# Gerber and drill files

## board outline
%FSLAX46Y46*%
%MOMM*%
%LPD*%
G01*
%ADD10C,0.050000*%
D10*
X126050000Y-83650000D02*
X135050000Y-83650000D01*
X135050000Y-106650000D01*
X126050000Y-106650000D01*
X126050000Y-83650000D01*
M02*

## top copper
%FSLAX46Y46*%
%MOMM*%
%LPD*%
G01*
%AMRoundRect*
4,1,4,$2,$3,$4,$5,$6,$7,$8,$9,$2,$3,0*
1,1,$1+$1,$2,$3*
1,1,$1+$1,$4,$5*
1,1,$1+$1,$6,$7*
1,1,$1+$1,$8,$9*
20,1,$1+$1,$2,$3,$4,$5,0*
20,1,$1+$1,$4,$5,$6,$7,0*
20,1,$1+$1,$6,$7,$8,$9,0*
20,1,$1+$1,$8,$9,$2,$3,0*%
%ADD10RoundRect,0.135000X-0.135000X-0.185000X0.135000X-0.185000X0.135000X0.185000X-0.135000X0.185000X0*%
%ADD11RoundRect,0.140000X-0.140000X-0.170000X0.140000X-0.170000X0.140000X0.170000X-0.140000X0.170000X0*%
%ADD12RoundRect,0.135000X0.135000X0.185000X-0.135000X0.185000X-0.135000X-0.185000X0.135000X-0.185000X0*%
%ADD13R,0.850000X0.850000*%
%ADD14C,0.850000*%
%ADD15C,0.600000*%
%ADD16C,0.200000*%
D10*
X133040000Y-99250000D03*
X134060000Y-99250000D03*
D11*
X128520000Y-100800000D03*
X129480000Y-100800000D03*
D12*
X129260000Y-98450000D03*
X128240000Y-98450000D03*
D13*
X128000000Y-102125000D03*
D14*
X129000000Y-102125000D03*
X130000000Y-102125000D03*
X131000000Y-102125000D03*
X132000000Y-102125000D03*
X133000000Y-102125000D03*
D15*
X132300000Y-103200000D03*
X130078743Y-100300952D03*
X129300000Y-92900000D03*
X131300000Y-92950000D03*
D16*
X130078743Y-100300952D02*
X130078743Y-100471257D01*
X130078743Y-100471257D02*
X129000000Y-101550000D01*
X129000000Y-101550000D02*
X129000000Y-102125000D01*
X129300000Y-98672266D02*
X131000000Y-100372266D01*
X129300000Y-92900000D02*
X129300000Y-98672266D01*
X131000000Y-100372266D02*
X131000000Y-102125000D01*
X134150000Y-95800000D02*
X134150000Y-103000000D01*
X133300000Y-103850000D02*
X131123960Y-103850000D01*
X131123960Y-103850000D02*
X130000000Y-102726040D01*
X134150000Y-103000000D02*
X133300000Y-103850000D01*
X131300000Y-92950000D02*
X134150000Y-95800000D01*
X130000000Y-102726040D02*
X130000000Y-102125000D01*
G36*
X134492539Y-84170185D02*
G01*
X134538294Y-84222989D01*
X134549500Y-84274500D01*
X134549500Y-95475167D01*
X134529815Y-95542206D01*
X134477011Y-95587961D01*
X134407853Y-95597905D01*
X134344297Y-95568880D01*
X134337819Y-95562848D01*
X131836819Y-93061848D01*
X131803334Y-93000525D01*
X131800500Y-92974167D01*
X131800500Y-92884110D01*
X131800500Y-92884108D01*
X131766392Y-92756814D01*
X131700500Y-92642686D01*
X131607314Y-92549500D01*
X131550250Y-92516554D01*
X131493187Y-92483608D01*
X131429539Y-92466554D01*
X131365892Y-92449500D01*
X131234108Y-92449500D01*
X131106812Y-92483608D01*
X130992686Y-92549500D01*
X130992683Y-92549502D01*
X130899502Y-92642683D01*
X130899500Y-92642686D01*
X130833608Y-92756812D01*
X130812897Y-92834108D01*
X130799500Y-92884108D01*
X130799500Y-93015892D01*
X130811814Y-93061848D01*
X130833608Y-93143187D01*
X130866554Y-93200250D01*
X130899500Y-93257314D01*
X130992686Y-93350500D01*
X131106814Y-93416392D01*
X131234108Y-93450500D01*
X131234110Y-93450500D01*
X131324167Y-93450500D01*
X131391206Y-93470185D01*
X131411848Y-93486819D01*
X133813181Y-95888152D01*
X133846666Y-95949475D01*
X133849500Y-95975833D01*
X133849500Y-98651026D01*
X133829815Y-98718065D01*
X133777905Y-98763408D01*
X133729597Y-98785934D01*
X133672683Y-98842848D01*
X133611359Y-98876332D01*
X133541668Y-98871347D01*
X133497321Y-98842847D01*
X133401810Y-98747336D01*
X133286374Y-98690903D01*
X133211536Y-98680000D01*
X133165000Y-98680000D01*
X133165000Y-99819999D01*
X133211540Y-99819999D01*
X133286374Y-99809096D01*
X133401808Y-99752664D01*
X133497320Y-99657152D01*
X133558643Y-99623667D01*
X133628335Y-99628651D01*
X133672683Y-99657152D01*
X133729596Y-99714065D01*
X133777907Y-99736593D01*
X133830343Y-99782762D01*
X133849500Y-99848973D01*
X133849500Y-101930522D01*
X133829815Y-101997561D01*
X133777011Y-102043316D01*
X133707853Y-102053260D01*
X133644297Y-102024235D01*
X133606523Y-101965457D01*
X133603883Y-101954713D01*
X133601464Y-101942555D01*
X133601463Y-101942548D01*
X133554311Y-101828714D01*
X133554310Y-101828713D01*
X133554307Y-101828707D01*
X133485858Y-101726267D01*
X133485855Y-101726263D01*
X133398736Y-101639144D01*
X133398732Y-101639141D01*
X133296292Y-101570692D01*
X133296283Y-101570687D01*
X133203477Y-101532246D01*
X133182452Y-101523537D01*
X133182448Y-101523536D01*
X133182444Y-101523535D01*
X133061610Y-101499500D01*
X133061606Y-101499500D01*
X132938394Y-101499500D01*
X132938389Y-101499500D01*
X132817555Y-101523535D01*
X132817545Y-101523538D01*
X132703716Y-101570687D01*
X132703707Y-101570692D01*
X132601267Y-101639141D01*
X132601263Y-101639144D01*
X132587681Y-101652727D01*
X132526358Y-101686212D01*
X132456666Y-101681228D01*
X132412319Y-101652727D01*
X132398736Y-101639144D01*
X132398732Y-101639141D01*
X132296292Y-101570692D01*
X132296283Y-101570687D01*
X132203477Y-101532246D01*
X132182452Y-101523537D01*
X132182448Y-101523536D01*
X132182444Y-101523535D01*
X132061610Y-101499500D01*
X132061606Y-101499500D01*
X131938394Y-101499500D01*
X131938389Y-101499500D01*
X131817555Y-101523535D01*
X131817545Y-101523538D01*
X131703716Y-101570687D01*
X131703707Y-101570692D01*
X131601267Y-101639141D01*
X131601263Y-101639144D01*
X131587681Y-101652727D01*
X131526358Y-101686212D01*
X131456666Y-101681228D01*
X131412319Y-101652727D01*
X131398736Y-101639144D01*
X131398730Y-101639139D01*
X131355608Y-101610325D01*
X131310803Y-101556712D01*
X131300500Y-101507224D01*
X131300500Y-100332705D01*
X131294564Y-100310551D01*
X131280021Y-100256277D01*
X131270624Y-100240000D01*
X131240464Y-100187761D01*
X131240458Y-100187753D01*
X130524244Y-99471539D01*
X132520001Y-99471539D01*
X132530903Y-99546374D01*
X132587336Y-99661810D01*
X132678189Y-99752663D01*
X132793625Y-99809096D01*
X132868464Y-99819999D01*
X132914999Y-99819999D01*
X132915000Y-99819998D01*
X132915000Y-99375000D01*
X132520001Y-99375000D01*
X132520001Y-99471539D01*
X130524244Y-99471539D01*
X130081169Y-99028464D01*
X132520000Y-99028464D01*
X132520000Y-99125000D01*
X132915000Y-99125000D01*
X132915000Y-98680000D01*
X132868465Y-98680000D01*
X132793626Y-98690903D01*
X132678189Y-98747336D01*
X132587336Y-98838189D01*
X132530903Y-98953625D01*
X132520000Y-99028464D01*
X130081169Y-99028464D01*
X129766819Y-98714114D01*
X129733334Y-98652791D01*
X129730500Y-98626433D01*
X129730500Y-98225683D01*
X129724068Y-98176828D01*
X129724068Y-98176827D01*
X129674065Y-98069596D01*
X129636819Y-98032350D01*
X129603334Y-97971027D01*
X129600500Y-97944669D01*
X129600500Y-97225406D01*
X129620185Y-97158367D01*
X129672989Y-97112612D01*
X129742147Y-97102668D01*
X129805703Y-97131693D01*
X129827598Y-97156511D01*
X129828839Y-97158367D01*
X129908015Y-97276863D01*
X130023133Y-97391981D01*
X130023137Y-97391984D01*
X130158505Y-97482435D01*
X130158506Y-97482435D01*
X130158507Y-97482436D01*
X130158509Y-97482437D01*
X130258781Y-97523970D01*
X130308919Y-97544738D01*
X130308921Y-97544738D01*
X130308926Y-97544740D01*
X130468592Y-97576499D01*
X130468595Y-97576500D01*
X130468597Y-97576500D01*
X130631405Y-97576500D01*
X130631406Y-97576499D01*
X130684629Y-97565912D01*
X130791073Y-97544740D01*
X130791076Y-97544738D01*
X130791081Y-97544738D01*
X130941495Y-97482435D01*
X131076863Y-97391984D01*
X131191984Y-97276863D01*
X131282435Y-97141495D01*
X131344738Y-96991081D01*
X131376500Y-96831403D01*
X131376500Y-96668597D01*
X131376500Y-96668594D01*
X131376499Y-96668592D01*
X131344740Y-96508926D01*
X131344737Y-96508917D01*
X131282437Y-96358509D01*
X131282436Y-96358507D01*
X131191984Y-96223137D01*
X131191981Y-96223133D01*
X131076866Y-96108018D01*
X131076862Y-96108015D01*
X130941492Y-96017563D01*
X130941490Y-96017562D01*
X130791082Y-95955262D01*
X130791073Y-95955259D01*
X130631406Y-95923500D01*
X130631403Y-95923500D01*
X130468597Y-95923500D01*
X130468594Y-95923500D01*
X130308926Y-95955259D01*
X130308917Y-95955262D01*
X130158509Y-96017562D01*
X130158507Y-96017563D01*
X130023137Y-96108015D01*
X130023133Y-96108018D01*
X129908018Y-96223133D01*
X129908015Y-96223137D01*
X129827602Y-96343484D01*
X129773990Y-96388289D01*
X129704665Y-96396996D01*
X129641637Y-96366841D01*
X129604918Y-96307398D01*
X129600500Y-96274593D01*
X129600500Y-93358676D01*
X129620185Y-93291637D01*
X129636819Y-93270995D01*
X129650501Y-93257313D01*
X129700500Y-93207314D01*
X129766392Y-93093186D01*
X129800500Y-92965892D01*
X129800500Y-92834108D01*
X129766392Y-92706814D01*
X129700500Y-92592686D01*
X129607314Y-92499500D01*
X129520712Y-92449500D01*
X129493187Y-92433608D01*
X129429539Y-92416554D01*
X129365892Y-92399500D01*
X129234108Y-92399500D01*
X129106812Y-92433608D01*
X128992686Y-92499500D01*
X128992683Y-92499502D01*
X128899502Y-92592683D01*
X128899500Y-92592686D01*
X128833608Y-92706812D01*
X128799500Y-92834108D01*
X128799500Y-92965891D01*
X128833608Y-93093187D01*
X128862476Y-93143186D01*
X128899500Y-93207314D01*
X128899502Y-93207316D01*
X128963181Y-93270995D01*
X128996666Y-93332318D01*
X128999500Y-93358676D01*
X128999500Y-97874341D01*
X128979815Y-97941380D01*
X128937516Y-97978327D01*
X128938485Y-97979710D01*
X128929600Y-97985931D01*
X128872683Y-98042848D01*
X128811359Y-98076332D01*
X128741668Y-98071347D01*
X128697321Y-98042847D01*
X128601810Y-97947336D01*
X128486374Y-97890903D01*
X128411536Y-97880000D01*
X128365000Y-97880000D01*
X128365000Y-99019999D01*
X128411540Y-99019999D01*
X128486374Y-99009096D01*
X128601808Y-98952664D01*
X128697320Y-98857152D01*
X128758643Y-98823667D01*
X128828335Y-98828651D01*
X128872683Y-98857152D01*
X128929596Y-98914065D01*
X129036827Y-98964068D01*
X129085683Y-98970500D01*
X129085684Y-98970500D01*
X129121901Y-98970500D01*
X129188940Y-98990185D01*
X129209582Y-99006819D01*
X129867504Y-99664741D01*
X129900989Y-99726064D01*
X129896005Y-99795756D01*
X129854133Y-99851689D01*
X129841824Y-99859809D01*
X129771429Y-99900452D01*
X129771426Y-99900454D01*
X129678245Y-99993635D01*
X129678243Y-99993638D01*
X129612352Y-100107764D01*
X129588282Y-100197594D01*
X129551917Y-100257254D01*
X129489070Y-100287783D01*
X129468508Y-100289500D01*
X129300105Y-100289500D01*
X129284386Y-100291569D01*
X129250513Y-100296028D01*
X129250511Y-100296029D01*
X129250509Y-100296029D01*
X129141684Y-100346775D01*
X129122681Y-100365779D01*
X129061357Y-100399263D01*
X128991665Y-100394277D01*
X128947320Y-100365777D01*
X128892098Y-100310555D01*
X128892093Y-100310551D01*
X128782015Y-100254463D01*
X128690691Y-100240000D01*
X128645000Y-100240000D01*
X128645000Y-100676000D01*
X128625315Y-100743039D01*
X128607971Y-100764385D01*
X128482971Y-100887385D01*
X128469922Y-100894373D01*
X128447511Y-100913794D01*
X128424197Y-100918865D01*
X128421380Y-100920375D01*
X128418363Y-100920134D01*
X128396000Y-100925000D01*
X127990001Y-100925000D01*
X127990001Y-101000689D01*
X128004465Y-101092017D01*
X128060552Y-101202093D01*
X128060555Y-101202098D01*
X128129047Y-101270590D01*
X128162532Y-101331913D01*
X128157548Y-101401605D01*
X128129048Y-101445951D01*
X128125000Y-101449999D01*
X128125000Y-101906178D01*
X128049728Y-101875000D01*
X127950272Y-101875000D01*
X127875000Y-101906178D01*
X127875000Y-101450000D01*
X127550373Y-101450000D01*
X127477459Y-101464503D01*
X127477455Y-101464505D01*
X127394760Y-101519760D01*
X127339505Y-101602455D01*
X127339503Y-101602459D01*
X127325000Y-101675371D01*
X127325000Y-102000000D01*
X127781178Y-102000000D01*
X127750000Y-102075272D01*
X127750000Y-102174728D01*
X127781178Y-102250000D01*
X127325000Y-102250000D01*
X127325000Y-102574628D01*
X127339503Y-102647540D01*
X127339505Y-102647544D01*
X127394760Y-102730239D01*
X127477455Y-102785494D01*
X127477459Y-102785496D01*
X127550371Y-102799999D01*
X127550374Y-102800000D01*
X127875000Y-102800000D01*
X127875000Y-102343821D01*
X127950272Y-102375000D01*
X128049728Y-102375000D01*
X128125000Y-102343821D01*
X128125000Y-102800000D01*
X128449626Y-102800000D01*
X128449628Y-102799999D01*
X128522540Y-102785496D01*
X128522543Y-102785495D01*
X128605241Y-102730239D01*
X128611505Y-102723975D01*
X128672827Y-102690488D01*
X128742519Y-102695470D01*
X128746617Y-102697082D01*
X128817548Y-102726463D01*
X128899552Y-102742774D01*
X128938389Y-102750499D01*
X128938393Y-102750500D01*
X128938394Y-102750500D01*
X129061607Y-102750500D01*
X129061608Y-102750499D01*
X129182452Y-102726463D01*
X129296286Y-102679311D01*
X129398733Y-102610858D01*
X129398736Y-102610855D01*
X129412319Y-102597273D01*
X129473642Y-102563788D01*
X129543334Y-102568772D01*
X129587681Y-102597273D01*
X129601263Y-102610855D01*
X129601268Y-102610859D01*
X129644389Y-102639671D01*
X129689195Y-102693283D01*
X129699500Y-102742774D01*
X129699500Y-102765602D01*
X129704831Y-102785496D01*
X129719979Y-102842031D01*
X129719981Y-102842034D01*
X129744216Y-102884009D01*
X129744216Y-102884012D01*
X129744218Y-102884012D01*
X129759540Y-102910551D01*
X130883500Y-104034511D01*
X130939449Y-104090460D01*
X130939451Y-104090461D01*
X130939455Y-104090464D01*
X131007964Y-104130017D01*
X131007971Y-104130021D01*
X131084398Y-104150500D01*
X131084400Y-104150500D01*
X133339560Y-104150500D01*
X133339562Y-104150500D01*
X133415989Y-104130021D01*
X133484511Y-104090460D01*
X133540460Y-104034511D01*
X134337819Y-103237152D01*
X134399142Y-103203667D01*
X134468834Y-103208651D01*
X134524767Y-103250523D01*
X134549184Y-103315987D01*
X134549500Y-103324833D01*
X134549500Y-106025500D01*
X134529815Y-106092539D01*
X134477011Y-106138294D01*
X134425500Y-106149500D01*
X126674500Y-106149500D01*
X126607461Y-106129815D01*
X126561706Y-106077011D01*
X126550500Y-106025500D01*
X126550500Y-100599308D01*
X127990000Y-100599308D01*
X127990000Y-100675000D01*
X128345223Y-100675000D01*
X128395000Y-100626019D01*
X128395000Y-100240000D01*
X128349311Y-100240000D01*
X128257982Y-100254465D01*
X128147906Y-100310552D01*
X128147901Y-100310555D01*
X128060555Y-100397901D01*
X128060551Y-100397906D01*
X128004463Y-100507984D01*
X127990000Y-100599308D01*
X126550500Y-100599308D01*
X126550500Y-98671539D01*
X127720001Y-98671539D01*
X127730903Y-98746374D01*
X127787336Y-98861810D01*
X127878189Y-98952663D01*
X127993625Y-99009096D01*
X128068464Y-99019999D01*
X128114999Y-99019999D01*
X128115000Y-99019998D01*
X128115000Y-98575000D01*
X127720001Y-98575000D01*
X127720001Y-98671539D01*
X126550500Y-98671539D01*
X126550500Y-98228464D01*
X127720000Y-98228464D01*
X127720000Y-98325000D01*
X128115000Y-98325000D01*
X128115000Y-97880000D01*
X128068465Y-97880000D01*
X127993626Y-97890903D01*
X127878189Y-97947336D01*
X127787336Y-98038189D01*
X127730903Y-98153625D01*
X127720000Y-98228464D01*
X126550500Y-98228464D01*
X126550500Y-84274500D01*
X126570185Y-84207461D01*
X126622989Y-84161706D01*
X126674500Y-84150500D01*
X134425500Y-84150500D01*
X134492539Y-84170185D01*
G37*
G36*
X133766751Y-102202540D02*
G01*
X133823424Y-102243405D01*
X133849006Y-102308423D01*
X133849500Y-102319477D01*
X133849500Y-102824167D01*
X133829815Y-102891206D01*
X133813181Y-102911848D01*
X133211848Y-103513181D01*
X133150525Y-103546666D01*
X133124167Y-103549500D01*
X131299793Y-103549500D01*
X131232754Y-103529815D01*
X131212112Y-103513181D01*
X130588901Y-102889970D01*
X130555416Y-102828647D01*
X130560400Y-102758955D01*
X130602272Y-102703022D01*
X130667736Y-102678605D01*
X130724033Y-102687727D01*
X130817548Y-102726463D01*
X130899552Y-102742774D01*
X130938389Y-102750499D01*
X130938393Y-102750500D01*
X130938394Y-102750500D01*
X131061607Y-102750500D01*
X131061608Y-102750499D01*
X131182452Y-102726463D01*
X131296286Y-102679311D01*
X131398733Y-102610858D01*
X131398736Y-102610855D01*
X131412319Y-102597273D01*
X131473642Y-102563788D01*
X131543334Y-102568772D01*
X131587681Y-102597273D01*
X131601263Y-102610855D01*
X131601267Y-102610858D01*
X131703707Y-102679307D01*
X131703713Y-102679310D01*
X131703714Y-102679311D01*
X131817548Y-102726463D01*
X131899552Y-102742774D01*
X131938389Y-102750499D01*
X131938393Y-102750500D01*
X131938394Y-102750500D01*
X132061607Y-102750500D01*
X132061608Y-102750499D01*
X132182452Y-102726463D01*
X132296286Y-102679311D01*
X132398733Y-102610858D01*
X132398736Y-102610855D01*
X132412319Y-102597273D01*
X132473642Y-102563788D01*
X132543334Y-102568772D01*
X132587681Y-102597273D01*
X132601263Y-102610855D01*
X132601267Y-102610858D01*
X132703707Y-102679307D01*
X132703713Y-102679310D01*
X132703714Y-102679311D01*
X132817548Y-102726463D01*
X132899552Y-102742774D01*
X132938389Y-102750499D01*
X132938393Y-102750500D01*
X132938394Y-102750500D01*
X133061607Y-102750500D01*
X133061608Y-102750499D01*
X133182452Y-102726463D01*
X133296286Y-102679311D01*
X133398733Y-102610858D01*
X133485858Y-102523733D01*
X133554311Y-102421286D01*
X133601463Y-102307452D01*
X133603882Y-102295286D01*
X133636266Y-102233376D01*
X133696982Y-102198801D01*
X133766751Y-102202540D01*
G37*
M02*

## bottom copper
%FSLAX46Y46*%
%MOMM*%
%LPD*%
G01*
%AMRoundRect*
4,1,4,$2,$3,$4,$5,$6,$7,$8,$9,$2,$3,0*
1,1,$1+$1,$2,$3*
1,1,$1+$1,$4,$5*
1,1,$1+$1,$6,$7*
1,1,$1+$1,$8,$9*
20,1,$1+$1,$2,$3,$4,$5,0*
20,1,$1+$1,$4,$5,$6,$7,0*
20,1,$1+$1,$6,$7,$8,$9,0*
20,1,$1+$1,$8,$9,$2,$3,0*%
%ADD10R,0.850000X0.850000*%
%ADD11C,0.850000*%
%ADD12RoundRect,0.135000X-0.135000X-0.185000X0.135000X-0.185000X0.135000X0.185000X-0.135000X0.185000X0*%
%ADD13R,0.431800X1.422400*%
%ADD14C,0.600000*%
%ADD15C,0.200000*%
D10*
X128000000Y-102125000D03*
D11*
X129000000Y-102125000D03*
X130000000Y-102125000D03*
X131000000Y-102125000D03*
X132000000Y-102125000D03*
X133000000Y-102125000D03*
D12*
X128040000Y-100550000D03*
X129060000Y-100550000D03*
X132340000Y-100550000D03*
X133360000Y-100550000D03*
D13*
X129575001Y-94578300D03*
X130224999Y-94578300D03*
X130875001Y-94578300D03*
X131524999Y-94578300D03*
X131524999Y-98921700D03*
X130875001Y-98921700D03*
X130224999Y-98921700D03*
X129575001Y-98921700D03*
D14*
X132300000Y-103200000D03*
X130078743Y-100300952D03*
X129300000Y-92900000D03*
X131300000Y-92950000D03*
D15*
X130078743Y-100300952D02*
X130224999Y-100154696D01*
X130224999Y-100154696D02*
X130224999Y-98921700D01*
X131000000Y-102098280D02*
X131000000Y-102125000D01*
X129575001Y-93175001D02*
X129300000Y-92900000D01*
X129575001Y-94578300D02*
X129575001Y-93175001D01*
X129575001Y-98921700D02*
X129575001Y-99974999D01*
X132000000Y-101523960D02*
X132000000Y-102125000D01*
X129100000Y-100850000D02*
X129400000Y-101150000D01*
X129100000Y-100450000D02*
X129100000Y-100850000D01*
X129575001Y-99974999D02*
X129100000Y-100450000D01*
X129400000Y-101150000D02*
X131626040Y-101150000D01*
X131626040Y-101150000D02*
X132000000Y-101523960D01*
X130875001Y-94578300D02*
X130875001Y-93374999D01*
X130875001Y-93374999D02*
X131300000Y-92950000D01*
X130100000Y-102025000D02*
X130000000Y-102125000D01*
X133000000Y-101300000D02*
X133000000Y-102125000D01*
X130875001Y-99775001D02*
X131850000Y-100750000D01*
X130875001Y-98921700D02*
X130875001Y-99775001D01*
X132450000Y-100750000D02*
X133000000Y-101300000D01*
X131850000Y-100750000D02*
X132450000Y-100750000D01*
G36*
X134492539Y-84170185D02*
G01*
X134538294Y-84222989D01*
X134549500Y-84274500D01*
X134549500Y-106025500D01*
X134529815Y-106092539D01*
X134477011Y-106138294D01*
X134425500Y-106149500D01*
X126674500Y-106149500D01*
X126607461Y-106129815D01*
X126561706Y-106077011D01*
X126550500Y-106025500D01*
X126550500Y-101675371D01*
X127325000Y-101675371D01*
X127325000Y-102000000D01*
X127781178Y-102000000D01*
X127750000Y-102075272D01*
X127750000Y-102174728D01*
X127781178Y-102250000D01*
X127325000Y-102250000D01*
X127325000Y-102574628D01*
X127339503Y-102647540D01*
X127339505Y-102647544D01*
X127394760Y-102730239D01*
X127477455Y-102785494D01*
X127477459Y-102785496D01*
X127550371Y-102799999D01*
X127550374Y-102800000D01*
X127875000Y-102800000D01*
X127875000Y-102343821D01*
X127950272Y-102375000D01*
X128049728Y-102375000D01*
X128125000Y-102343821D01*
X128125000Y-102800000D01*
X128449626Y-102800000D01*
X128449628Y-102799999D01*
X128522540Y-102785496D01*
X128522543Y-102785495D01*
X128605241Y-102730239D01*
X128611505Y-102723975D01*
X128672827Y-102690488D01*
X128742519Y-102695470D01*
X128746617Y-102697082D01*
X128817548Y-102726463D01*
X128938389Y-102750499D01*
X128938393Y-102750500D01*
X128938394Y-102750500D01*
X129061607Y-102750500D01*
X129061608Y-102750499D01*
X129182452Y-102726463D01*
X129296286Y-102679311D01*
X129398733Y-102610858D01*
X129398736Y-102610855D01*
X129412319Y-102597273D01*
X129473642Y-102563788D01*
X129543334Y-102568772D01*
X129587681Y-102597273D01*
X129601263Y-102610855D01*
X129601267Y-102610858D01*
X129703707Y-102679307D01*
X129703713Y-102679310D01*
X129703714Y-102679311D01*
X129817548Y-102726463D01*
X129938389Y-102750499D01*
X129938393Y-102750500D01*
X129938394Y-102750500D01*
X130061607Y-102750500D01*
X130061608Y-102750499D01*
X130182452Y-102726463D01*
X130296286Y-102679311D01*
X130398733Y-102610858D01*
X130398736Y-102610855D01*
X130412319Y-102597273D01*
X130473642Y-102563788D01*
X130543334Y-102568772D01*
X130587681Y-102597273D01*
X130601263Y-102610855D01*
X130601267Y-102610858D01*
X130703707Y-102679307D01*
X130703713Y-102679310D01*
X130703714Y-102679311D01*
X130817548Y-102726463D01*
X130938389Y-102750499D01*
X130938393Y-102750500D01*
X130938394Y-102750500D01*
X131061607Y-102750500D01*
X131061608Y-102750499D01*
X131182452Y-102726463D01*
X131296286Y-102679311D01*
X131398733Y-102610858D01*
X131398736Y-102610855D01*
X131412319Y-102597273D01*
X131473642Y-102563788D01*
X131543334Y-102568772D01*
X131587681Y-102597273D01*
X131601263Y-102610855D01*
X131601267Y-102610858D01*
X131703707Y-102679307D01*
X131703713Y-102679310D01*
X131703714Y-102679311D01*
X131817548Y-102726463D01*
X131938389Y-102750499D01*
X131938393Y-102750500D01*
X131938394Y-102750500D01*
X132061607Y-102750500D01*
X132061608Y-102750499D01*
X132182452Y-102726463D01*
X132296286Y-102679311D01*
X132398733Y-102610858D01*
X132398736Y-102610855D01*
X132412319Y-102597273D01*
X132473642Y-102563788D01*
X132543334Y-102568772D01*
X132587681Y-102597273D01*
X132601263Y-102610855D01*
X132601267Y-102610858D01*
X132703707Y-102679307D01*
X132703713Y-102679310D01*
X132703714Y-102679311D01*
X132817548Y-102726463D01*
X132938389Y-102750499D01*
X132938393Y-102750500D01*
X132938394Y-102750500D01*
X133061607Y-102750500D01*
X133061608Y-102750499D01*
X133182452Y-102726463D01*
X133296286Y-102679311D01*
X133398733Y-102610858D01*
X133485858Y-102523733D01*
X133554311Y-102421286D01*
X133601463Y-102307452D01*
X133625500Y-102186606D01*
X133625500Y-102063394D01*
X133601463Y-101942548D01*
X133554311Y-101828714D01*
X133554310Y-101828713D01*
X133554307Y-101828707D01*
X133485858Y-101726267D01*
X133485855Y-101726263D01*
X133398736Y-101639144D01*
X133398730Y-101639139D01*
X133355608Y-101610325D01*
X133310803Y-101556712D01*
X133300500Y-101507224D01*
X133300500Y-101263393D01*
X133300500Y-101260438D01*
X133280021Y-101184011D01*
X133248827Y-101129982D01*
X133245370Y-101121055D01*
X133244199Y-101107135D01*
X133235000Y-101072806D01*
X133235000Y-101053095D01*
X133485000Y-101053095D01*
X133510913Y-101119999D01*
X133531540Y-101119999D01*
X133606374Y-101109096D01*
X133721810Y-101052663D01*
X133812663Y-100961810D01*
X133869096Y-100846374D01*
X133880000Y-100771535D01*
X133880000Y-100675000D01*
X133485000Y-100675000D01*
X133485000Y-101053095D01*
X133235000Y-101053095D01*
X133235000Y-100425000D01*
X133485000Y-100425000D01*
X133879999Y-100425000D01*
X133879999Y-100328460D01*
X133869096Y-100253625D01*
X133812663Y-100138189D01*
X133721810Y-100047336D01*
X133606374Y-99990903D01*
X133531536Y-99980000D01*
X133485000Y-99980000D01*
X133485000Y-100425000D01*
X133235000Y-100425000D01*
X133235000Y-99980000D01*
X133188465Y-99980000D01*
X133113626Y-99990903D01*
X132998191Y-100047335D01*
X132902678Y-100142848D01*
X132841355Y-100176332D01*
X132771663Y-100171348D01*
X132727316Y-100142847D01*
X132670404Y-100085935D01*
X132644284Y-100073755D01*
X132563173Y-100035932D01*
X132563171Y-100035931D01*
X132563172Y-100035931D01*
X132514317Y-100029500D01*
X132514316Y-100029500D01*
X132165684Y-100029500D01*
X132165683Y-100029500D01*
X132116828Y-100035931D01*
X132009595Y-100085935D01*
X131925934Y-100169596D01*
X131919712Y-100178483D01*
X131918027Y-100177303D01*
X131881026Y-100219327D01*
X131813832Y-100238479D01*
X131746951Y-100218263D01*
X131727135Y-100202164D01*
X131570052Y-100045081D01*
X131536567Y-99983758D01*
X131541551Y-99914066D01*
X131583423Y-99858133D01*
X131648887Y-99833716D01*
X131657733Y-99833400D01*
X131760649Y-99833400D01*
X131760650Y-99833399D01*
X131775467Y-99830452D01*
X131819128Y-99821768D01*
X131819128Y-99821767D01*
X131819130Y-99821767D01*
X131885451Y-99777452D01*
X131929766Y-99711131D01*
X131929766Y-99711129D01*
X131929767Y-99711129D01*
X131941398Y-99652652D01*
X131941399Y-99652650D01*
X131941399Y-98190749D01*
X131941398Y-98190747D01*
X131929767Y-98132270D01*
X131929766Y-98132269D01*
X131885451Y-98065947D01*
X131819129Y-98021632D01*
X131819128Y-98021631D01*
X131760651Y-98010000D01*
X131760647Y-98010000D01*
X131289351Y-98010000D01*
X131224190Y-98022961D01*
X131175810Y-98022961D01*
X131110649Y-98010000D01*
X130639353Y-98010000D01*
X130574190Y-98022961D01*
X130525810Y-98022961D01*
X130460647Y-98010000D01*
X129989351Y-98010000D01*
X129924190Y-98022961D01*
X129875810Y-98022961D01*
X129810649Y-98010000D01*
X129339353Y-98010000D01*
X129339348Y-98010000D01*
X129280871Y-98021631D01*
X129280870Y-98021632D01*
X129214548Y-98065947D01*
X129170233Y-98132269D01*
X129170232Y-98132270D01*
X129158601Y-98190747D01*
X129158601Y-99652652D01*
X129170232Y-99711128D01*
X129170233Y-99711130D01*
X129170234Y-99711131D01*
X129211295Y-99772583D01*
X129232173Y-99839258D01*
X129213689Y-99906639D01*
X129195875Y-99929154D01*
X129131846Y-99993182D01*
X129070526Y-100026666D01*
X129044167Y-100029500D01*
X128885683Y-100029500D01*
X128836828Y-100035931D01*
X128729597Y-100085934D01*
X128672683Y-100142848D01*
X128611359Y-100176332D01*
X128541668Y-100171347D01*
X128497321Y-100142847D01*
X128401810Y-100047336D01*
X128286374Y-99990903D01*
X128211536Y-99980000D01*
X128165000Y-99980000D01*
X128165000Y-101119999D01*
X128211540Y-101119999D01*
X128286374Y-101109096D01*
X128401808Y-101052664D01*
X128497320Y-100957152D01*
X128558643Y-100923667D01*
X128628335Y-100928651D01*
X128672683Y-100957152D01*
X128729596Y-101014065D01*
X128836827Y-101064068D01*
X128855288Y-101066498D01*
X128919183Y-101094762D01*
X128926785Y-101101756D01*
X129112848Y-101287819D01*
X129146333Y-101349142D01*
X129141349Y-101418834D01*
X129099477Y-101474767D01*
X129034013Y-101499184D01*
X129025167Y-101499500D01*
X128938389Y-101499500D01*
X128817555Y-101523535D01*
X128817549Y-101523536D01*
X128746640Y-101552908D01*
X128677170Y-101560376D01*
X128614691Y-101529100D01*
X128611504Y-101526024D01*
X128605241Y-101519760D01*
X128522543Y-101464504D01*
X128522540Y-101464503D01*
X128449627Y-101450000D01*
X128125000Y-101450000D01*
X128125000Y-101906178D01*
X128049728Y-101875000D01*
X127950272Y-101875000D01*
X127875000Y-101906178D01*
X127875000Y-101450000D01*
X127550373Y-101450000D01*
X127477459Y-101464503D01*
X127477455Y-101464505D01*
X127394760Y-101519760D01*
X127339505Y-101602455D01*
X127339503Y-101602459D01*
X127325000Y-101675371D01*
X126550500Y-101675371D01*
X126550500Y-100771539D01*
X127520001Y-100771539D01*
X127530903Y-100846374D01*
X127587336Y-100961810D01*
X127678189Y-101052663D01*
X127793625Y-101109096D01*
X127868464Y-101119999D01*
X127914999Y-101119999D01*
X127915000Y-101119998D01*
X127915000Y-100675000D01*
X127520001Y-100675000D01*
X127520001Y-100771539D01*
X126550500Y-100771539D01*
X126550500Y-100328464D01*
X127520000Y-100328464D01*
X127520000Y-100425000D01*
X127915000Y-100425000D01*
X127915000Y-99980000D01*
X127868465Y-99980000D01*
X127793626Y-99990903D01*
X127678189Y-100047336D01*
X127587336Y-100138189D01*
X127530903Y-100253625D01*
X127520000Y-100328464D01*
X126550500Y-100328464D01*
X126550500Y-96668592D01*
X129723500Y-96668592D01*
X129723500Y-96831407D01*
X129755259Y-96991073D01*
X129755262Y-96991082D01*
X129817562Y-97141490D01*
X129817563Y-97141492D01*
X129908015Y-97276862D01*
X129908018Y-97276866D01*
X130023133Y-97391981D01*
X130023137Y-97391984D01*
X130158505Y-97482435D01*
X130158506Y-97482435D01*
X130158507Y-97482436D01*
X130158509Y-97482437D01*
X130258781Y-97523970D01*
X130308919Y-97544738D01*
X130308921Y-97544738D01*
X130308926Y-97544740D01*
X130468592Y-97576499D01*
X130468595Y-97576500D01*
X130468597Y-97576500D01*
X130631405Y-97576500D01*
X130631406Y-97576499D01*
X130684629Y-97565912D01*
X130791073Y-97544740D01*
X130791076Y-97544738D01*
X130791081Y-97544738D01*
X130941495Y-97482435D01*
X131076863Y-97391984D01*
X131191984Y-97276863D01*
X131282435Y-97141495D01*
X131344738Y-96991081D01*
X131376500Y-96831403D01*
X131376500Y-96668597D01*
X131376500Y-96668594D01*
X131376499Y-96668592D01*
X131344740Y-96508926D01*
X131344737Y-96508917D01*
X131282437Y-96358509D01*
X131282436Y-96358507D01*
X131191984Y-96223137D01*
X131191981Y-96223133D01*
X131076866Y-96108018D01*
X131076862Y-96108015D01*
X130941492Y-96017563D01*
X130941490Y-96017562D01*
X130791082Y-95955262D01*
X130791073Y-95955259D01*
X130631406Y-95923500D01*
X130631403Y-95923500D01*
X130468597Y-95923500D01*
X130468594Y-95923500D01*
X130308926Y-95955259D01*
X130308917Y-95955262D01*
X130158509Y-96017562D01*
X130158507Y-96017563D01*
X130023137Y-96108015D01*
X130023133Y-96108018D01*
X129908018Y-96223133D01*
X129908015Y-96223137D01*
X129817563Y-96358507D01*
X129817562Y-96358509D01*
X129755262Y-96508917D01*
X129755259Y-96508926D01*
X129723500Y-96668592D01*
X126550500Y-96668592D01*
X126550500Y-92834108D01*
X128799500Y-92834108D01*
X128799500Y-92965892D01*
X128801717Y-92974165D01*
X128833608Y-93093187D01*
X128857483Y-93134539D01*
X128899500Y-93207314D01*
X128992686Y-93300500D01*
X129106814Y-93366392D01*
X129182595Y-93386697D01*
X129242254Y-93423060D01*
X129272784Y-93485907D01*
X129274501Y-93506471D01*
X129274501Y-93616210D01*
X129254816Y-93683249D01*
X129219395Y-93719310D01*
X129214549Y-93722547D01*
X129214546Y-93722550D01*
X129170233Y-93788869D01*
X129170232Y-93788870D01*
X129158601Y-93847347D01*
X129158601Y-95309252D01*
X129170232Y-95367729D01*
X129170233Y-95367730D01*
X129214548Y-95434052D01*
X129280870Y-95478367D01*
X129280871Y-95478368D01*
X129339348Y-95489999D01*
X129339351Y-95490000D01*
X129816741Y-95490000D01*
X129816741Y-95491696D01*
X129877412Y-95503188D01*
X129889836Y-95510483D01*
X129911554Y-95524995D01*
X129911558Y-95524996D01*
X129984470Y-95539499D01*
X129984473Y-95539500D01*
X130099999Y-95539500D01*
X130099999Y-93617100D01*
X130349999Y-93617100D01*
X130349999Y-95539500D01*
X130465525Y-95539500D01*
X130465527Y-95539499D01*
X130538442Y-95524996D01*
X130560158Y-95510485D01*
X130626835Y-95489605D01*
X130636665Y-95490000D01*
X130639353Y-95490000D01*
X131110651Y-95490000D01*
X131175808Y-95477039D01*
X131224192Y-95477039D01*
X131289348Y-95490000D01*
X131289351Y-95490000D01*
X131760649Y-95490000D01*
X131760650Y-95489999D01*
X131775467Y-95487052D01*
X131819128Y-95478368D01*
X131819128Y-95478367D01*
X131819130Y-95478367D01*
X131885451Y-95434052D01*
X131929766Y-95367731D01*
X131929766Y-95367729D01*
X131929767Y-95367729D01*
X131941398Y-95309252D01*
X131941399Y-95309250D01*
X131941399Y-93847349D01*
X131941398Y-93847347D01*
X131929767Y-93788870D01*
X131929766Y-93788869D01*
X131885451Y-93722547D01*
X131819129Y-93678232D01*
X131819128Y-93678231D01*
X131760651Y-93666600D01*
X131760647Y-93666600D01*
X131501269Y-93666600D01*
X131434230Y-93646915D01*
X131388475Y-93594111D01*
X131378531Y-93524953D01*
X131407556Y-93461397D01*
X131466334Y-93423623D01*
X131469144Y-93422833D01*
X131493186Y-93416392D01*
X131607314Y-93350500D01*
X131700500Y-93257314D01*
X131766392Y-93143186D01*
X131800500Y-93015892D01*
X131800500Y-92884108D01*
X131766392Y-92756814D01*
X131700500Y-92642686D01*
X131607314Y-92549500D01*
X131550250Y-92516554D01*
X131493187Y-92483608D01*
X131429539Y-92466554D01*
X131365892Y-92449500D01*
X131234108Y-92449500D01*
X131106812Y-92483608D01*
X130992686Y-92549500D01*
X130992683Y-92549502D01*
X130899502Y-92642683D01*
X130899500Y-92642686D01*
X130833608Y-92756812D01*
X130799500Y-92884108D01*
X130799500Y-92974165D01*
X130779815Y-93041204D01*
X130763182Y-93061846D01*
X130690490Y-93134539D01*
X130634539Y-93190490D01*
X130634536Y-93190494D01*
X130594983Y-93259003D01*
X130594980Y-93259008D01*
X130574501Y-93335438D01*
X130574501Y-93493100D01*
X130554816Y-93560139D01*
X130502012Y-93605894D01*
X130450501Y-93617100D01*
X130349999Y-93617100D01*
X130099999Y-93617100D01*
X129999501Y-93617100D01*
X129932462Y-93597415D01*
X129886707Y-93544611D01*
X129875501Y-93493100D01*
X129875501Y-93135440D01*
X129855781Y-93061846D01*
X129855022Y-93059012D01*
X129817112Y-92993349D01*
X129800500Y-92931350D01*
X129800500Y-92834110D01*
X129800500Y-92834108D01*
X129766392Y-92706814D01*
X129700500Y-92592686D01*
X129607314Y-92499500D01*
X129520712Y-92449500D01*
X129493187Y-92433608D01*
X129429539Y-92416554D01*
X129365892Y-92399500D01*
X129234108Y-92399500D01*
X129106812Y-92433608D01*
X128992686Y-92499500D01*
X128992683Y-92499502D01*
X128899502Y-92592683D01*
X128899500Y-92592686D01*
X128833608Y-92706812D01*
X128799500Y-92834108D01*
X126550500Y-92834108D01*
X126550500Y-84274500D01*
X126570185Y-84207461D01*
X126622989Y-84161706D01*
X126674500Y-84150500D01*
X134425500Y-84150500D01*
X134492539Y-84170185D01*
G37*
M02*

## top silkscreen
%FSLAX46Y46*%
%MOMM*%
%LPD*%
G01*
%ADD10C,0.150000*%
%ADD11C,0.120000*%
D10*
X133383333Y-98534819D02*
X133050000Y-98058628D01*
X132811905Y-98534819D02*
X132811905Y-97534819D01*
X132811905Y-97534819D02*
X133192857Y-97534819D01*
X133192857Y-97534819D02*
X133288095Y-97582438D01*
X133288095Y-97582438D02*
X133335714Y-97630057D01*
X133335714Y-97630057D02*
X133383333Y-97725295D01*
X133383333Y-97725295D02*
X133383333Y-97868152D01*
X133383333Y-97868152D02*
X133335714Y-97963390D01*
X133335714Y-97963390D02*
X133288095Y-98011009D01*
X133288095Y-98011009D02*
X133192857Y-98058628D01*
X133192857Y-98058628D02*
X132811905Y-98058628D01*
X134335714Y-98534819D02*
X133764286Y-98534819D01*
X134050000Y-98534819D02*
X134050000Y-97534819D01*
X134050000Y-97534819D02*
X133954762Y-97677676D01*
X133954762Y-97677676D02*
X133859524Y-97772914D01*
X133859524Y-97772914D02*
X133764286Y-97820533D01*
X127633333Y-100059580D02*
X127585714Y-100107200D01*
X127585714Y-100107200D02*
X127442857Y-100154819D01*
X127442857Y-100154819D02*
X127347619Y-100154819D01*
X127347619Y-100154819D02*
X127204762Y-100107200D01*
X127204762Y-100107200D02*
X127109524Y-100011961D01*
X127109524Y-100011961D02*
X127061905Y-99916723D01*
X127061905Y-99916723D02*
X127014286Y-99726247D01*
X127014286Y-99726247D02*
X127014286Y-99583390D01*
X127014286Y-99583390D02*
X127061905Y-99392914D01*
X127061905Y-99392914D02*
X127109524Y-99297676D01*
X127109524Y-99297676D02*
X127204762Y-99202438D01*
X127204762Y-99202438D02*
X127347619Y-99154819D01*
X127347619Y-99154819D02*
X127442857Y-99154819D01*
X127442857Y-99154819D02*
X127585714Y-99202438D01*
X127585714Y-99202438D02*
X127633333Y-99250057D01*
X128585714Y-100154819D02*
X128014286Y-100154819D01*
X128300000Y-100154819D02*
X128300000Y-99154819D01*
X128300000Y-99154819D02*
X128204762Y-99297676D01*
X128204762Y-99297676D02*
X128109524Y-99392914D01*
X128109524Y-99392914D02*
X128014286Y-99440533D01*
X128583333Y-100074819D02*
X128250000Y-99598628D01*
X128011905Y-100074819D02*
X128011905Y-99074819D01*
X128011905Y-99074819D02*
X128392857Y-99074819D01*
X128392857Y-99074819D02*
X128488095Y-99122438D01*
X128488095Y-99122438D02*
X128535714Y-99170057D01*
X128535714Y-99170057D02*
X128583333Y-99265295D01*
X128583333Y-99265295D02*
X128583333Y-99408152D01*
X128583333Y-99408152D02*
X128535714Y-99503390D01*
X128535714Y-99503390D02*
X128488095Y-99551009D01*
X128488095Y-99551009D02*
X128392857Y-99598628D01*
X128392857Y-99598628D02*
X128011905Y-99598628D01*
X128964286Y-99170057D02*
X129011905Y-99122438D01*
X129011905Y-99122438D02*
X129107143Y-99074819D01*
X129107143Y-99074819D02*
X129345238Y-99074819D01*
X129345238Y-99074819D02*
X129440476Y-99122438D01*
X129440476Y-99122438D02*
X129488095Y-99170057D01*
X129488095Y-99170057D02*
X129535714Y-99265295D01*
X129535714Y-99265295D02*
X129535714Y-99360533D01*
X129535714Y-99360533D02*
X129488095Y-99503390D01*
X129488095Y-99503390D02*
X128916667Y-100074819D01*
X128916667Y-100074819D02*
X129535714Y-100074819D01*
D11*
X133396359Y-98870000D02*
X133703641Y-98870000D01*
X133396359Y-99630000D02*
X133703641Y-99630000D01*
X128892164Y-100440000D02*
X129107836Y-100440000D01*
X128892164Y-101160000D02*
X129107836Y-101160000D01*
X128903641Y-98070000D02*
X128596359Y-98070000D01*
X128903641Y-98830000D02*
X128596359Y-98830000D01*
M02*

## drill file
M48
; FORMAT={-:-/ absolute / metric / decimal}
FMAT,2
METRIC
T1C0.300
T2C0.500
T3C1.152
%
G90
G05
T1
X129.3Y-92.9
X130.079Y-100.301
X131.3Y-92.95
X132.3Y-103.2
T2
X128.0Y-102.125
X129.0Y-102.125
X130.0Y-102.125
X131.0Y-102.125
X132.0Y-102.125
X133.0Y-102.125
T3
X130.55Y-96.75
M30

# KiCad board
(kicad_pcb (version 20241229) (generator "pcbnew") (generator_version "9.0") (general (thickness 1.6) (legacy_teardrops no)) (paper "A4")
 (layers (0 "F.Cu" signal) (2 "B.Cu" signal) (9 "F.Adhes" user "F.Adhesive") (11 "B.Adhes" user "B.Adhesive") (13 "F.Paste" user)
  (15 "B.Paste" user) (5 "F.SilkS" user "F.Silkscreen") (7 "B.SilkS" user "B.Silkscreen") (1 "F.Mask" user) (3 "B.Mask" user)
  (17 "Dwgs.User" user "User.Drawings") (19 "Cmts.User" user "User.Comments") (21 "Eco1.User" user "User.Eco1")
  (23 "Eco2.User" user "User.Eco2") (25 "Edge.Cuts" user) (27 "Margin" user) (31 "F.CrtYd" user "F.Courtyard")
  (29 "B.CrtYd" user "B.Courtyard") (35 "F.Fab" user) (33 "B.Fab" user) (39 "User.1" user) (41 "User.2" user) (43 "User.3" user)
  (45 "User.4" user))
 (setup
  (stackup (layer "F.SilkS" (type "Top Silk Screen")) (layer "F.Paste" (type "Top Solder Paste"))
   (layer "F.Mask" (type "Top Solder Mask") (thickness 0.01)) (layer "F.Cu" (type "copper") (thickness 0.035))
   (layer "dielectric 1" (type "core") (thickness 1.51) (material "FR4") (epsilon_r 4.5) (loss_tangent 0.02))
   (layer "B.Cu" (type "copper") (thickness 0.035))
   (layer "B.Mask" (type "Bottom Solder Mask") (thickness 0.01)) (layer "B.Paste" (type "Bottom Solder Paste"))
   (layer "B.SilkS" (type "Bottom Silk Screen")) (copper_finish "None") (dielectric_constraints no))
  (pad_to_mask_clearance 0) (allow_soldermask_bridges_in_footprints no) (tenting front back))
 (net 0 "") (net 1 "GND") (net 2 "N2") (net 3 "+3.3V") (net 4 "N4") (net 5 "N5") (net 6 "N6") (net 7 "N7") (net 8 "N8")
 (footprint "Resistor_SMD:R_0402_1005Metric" (layer "F.Cu") (at 133.55 99.25)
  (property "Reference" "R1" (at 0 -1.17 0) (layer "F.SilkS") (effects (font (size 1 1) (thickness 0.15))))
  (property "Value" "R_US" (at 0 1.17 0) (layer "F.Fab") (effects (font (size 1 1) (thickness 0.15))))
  (fp_line (start -0.153641 -0.38) (end 0.153641 -0.38) (stroke (width 0.12) (type solid)) (layer "F.SilkS"))
  (fp_line (start -0.153641 0.38) (end 0.153641 0.38) (stroke (width 0.12) (type solid)) (layer "F.SilkS"))
  (pad "1" smd roundrect (at -0.51 0) (size 0.54 0.64) (layers "F.Cu" "F.Mask" "F.Paste") (roundrect_rratio 0.25) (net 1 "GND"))
  (pad "2" smd roundrect (at 0.51 0) (size 0.54 0.64) (layers "F.Cu" "F.Mask" "F.Paste") (roundrect_rratio 0.25) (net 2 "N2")))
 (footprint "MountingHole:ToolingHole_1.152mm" (layer "F.Cu") (at 130.55 96.75)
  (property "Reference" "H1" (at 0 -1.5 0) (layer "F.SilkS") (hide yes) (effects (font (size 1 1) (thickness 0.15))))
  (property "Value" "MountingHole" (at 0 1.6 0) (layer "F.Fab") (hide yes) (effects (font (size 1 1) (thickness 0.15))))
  (pad "" np_thru_hole circle (at 0 0) (size 1.152 1.152) (drill 1.152) (layers "*.Cu" "*.Mask") (solder_mask_margin 0.074))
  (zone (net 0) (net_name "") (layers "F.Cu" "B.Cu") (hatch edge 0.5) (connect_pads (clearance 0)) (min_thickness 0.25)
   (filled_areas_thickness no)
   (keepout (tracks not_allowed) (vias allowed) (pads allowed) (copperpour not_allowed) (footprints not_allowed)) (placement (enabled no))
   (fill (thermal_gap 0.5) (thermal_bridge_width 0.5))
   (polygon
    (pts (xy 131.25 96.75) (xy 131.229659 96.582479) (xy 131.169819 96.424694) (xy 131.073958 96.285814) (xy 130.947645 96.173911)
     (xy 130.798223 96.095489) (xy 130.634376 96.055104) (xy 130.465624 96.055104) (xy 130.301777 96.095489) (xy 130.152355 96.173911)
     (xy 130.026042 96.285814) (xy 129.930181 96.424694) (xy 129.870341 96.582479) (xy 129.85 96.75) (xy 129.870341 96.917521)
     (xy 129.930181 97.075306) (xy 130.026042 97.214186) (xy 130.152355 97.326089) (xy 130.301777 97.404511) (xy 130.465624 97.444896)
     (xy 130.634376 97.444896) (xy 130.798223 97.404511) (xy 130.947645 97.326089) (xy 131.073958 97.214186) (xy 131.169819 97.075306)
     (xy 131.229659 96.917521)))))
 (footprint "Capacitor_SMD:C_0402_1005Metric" (layer "F.Cu") (at 129 100.8)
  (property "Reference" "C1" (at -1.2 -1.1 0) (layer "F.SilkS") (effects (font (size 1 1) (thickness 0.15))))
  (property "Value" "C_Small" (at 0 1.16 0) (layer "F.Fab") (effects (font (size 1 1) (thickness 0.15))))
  (fp_line (start -0.107836 -0.36) (end 0.107836 -0.36) (stroke (width 0.12) (type solid)) (layer "F.SilkS"))
  (fp_line (start -0.107836 0.36) (end 0.107836 0.36) (stroke (width 0.12) (type solid)) (layer "F.SilkS"))
  (pad "1" smd roundrect (at -0.48 0) (size 0.56 0.62) (layers "F.Cu" "F.Mask" "F.Paste") (roundrect_rratio 0.25) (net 1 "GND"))
  (pad "2" smd roundrect (at 0.48 0) (size 0.56 0.62) (layers "F.Cu" "F.Mask" "F.Paste") (roundrect_rratio 0.25) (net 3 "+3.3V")))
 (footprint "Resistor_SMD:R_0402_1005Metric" (layer "F.Cu") (at 128.75 98.45 180)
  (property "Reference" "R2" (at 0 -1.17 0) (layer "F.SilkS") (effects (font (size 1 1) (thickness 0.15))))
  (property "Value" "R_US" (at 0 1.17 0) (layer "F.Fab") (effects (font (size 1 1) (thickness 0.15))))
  (fp_line (start -0.153641 0.38) (end 0.153641 0.38) (stroke (width 0.12) (type solid)) (layer "F.SilkS"))
  (fp_line (start -0.153641 -0.38) (end 0.153641 -0.38) (stroke (width 0.12) (type solid)) (layer "F.SilkS"))
  (pad "1" smd roundrect (at -0.51 0 180) (size 0.54 0.64) (layers "F.Cu" "F.Mask" "F.Paste") (roundrect_rratio 0.25) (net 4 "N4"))
  (pad "2" smd roundrect (at 0.51 0 180) (size 0.54 0.64) (layers "F.Cu" "F.Mask" "F.Paste") (roundrect_rratio 0.25) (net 1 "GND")))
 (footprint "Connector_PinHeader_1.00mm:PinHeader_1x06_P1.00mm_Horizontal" (layer "B.Cu") (at 128 102.125 -90)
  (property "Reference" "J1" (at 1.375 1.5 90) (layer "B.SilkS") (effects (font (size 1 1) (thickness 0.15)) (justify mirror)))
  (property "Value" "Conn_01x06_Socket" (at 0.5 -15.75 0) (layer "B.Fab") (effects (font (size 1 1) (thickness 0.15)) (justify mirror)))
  (pad "1" thru_hole rect (at 0 0 270) (size 0.85 0.85) (drill 0.5) (layers "*.Cu" "*.Mask") (remove_unused_layers no) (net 1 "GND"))
  (pad "2" thru_hole circle (at 0 -1 270) (size 0.85 0.85) (drill 0.5) (layers "*.Cu" "*.Mask") (remove_unused_layers no) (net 3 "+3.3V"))
  (pad "3" thru_hole circle (at 0 -2 270) (size 0.85 0.85) (drill 0.5) (layers "*.Cu" "*.Mask") (remove_unused_layers no) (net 2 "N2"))
  (pad "4" thru_hole circle (at 0 -3 270) (size 0.85 0.85) (drill 0.5) (layers "*.Cu" "*.Mask") (remove_unused_layers no) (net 4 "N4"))
  (pad "5" thru_hole circle (at 0 -4 270) (size 0.85 0.85) (drill 0.5) (layers "*.Cu" "*.Mask") (remove_unused_layers no) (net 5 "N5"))
  (pad "6" thru_hole circle (at 0 -5 270) (size 0.85 0.85) (drill 0.5) (layers "*.Cu" "*.Mask") (remove_unused_layers no) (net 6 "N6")))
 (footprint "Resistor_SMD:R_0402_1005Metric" (layer "B.Cu") (at 128.55 100.55)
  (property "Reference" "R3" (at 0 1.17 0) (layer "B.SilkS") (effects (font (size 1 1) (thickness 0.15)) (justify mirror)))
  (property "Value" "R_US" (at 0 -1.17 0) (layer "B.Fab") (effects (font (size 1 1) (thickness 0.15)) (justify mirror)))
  (pad "1" smd roundrect (at -0.51 0) (size 0.54 0.64) (layers "B.Cu" "B.Mask" "B.Paste") (roundrect_rratio 0.25) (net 1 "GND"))
  (pad "2" smd roundrect (at 0.51 0) (size 0.54 0.64) (layers "B.Cu" "B.Mask" "B.Paste") (roundrect_rratio 0.25) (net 5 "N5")))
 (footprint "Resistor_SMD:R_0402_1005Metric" (layer "B.Cu") (at 132.85 100.55)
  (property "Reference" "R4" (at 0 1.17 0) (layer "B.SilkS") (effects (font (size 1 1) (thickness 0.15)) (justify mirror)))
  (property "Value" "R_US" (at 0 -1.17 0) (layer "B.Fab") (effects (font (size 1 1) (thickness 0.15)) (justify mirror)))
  (pad "1" smd roundrect (at -0.51 0) (size 0.54 0.64) (layers "B.Cu" "B.Mask" "B.Paste") (roundrect_rratio 0.25) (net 6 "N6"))
  (pad "2" smd roundrect (at 0.51 0) (size 0.54 0.64) (layers "B.Cu" "B.Mask" "B.Paste") (roundrect_rratio 0.25) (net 1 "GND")))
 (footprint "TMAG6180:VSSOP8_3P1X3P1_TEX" (layer "B.Cu") (at 130.55 96.75 -90)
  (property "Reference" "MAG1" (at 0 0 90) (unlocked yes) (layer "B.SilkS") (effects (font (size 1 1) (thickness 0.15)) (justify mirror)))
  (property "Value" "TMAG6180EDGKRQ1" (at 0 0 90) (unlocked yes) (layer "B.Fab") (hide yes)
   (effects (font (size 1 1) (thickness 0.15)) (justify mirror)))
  (pad "1" smd rect (at -2.1717 0.974999 270) (size 1.4224 0.4318) (layers "B.Cu" "B.Mask" "B.Paste") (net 4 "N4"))
  (pad "2" smd rect (at -2.1717 0.325001 270) (size 1.4224 0.4318) (layers "B.Cu" "B.Mask" "B.Paste") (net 1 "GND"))
  (pad "3" smd rect (at -2.1717 -0.325001 270) (size 1.4224 0.4318) (layers "B.Cu" "B.Mask" "B.Paste") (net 2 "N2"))
  (pad "4" smd rect (at -2.1717 -0.974999 270) (size 1.4224 0.4318) (layers "B.Cu" "B.Mask" "B.Paste") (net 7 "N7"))
  (pad "5" smd rect (at 2.1717 -0.974999 270) (size 1.4224 0.4318) (layers "B.Cu" "B.Mask" "B.Paste") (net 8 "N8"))
  (pad "6" smd rect (at 2.1717 -0.325001 270) (size 1.4224 0.4318) (layers "B.Cu" "B.Mask" "B.Paste") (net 6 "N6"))
  (pad "7" smd rect (at 2.1717 0.325001 270) (size 1.4224 0.4318) (layers "B.Cu" "B.Mask" "B.Paste") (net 3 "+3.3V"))
  (pad "8" smd rect (at 2.1717 0.974999 270) (size 1.4224 0.4318) (layers "B.Cu" "B.Mask" "B.Paste") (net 5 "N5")))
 (gr_rect (start 126.05 83.65) (end 135.05 106.65) (stroke (width 0.05) (type solid)) (fill no) (locked yes) (layer "Edge.Cuts"))
 (via (at 132.3 103.2) (size 0.6) (drill 0.3) (layers "F.Cu" "B.Cu") (free yes) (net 1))
 (segment (start 130.078743 100.300952) (end 130.078743 100.471257) (width 0.2) (layer "F.Cu") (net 3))
 (segment (start 130.078743 100.471257) (end 129 101.55) (width 0.2) (layer "F.Cu") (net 3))
 (segment (start 129 101.55) (end 129 102.125) (width 0.2) (layer "F.Cu") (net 3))
 (via (at 130.078743 100.300952) (size 0.6) (drill 0.3) (layers "F.Cu" "B.Cu") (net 3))
 (segment (start 130.078743 100.300952) (end 130.224999 100.154696) (width 0.2) (layer "B.Cu") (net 3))
 (segment (start 130.224999 100.154696) (end 130.224999 98.9217) (width 0.2) (layer "B.Cu") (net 3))
 (segment (start 129.3 98.672266) (end 131 100.372266) (width 0.2) (layer "F.Cu") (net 4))
 (segment (start 129.3 92.9) (end 129.3 98.672266) (width 0.2) (layer "F.Cu") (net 4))
 (segment (start 131 100.372266) (end 131 102.125) (width 0.2) (layer "F.Cu") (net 4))
 (via (at 129.3 92.9) (size 0.6) (drill 0.3) (layers "F.Cu" "B.Cu") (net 4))
 (segment (start 131 102.09828) (end 131 102.125) (width 0.2) (layer "B.Cu") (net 4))
 (segment (start 129.575001 93.175001) (end 129.3 92.9) (width 0.2) (layer "B.Cu") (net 4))
 (segment (start 129.575001 94.5783) (end 129.575001 93.175001) (width 0.2) (layer "B.Cu") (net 4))
 (segment (start 129.575001 98.9217) (end 129.575001 99.974999) (width 0.2) (layer "B.Cu") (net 5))
 (segment (start 132 101.52396) (end 132 102.125) (width 0.2) (layer "B.Cu") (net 5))
 (segment (start 129.1 100.85) (end 129.4 101.15) (width 0.2) (layer "B.Cu") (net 5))
 (segment (start 129.1 100.45) (end 129.1 100.85) (width 0.2) (layer "B.Cu") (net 5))
 (segment (start 129.575001 99.974999) (end 129.1 100.45) (width 0.2) (layer "B.Cu") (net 5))
 (segment (start 129.4 101.15) (end 131.62604 101.15) (width 0.2) (layer "B.Cu") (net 5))
 (segment (start 131.62604 101.15) (end 132 101.52396) (width 0.2) (layer "B.Cu") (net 5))
 (segment (start 134.15 95.8) (end 134.15 103) (width 0.2) (layer "F.Cu") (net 2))
 (segment (start 133.3 103.85) (end 131.12396 103.85) (width 0.2) (layer "F.Cu") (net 2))
 (segment (start 131.12396 103.85) (end 130 102.72604) (width 0.2) (layer "F.Cu") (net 2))
 (segment (start 134.15 103) (end 133.3 103.85) (width 0.2) (layer "F.Cu") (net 2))
 (segment (start 131.3 92.95) (end 134.15 95.8) (width 0.2) (layer "F.Cu") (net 2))
 (segment (start 130 102.72604) (end 130 102.125) (width 0.2) (layer "F.Cu") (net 2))
 (via (at 131.3 92.95) (size 0.6) (drill 0.3) (layers "F.Cu" "B.Cu") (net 2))
 (segment (start 130.875001 94.5783) (end 130.875001 93.374999) (width 0.2) (layer "B.Cu") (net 2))
 (segment (start 130.875001 93.374999) (end 131.3 92.95) (width 0.2) (layer "B.Cu") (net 2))
 (segment (start 130.1 102.025) (end 130 102.125) (width 0.2) (layer "B.Cu") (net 2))
 (segment (start 133 101.3) (end 133 102.125) (width 0.2) (layer "B.Cu") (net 6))
 (segment (start 130.875001 99.775001) (end 131.85 100.75) (width 0.2) (layer "B.Cu") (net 6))
 (segment (start 130.875001 98.9217) (end 130.875001 99.775001) (width 0.2) (layer "B.Cu") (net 6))
 (segment (start 132.45 100.75) (end 133 101.3) (width 0.2) (layer "B.Cu") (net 6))
 (segment (start 131.85 100.75) (end 132.45 100.75) (width 0.2) (layer "B.Cu") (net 6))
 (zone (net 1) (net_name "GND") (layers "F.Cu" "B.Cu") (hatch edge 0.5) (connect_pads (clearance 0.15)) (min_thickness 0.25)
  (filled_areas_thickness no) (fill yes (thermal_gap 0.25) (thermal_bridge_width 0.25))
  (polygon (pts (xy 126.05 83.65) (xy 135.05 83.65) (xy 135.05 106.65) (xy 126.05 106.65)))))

